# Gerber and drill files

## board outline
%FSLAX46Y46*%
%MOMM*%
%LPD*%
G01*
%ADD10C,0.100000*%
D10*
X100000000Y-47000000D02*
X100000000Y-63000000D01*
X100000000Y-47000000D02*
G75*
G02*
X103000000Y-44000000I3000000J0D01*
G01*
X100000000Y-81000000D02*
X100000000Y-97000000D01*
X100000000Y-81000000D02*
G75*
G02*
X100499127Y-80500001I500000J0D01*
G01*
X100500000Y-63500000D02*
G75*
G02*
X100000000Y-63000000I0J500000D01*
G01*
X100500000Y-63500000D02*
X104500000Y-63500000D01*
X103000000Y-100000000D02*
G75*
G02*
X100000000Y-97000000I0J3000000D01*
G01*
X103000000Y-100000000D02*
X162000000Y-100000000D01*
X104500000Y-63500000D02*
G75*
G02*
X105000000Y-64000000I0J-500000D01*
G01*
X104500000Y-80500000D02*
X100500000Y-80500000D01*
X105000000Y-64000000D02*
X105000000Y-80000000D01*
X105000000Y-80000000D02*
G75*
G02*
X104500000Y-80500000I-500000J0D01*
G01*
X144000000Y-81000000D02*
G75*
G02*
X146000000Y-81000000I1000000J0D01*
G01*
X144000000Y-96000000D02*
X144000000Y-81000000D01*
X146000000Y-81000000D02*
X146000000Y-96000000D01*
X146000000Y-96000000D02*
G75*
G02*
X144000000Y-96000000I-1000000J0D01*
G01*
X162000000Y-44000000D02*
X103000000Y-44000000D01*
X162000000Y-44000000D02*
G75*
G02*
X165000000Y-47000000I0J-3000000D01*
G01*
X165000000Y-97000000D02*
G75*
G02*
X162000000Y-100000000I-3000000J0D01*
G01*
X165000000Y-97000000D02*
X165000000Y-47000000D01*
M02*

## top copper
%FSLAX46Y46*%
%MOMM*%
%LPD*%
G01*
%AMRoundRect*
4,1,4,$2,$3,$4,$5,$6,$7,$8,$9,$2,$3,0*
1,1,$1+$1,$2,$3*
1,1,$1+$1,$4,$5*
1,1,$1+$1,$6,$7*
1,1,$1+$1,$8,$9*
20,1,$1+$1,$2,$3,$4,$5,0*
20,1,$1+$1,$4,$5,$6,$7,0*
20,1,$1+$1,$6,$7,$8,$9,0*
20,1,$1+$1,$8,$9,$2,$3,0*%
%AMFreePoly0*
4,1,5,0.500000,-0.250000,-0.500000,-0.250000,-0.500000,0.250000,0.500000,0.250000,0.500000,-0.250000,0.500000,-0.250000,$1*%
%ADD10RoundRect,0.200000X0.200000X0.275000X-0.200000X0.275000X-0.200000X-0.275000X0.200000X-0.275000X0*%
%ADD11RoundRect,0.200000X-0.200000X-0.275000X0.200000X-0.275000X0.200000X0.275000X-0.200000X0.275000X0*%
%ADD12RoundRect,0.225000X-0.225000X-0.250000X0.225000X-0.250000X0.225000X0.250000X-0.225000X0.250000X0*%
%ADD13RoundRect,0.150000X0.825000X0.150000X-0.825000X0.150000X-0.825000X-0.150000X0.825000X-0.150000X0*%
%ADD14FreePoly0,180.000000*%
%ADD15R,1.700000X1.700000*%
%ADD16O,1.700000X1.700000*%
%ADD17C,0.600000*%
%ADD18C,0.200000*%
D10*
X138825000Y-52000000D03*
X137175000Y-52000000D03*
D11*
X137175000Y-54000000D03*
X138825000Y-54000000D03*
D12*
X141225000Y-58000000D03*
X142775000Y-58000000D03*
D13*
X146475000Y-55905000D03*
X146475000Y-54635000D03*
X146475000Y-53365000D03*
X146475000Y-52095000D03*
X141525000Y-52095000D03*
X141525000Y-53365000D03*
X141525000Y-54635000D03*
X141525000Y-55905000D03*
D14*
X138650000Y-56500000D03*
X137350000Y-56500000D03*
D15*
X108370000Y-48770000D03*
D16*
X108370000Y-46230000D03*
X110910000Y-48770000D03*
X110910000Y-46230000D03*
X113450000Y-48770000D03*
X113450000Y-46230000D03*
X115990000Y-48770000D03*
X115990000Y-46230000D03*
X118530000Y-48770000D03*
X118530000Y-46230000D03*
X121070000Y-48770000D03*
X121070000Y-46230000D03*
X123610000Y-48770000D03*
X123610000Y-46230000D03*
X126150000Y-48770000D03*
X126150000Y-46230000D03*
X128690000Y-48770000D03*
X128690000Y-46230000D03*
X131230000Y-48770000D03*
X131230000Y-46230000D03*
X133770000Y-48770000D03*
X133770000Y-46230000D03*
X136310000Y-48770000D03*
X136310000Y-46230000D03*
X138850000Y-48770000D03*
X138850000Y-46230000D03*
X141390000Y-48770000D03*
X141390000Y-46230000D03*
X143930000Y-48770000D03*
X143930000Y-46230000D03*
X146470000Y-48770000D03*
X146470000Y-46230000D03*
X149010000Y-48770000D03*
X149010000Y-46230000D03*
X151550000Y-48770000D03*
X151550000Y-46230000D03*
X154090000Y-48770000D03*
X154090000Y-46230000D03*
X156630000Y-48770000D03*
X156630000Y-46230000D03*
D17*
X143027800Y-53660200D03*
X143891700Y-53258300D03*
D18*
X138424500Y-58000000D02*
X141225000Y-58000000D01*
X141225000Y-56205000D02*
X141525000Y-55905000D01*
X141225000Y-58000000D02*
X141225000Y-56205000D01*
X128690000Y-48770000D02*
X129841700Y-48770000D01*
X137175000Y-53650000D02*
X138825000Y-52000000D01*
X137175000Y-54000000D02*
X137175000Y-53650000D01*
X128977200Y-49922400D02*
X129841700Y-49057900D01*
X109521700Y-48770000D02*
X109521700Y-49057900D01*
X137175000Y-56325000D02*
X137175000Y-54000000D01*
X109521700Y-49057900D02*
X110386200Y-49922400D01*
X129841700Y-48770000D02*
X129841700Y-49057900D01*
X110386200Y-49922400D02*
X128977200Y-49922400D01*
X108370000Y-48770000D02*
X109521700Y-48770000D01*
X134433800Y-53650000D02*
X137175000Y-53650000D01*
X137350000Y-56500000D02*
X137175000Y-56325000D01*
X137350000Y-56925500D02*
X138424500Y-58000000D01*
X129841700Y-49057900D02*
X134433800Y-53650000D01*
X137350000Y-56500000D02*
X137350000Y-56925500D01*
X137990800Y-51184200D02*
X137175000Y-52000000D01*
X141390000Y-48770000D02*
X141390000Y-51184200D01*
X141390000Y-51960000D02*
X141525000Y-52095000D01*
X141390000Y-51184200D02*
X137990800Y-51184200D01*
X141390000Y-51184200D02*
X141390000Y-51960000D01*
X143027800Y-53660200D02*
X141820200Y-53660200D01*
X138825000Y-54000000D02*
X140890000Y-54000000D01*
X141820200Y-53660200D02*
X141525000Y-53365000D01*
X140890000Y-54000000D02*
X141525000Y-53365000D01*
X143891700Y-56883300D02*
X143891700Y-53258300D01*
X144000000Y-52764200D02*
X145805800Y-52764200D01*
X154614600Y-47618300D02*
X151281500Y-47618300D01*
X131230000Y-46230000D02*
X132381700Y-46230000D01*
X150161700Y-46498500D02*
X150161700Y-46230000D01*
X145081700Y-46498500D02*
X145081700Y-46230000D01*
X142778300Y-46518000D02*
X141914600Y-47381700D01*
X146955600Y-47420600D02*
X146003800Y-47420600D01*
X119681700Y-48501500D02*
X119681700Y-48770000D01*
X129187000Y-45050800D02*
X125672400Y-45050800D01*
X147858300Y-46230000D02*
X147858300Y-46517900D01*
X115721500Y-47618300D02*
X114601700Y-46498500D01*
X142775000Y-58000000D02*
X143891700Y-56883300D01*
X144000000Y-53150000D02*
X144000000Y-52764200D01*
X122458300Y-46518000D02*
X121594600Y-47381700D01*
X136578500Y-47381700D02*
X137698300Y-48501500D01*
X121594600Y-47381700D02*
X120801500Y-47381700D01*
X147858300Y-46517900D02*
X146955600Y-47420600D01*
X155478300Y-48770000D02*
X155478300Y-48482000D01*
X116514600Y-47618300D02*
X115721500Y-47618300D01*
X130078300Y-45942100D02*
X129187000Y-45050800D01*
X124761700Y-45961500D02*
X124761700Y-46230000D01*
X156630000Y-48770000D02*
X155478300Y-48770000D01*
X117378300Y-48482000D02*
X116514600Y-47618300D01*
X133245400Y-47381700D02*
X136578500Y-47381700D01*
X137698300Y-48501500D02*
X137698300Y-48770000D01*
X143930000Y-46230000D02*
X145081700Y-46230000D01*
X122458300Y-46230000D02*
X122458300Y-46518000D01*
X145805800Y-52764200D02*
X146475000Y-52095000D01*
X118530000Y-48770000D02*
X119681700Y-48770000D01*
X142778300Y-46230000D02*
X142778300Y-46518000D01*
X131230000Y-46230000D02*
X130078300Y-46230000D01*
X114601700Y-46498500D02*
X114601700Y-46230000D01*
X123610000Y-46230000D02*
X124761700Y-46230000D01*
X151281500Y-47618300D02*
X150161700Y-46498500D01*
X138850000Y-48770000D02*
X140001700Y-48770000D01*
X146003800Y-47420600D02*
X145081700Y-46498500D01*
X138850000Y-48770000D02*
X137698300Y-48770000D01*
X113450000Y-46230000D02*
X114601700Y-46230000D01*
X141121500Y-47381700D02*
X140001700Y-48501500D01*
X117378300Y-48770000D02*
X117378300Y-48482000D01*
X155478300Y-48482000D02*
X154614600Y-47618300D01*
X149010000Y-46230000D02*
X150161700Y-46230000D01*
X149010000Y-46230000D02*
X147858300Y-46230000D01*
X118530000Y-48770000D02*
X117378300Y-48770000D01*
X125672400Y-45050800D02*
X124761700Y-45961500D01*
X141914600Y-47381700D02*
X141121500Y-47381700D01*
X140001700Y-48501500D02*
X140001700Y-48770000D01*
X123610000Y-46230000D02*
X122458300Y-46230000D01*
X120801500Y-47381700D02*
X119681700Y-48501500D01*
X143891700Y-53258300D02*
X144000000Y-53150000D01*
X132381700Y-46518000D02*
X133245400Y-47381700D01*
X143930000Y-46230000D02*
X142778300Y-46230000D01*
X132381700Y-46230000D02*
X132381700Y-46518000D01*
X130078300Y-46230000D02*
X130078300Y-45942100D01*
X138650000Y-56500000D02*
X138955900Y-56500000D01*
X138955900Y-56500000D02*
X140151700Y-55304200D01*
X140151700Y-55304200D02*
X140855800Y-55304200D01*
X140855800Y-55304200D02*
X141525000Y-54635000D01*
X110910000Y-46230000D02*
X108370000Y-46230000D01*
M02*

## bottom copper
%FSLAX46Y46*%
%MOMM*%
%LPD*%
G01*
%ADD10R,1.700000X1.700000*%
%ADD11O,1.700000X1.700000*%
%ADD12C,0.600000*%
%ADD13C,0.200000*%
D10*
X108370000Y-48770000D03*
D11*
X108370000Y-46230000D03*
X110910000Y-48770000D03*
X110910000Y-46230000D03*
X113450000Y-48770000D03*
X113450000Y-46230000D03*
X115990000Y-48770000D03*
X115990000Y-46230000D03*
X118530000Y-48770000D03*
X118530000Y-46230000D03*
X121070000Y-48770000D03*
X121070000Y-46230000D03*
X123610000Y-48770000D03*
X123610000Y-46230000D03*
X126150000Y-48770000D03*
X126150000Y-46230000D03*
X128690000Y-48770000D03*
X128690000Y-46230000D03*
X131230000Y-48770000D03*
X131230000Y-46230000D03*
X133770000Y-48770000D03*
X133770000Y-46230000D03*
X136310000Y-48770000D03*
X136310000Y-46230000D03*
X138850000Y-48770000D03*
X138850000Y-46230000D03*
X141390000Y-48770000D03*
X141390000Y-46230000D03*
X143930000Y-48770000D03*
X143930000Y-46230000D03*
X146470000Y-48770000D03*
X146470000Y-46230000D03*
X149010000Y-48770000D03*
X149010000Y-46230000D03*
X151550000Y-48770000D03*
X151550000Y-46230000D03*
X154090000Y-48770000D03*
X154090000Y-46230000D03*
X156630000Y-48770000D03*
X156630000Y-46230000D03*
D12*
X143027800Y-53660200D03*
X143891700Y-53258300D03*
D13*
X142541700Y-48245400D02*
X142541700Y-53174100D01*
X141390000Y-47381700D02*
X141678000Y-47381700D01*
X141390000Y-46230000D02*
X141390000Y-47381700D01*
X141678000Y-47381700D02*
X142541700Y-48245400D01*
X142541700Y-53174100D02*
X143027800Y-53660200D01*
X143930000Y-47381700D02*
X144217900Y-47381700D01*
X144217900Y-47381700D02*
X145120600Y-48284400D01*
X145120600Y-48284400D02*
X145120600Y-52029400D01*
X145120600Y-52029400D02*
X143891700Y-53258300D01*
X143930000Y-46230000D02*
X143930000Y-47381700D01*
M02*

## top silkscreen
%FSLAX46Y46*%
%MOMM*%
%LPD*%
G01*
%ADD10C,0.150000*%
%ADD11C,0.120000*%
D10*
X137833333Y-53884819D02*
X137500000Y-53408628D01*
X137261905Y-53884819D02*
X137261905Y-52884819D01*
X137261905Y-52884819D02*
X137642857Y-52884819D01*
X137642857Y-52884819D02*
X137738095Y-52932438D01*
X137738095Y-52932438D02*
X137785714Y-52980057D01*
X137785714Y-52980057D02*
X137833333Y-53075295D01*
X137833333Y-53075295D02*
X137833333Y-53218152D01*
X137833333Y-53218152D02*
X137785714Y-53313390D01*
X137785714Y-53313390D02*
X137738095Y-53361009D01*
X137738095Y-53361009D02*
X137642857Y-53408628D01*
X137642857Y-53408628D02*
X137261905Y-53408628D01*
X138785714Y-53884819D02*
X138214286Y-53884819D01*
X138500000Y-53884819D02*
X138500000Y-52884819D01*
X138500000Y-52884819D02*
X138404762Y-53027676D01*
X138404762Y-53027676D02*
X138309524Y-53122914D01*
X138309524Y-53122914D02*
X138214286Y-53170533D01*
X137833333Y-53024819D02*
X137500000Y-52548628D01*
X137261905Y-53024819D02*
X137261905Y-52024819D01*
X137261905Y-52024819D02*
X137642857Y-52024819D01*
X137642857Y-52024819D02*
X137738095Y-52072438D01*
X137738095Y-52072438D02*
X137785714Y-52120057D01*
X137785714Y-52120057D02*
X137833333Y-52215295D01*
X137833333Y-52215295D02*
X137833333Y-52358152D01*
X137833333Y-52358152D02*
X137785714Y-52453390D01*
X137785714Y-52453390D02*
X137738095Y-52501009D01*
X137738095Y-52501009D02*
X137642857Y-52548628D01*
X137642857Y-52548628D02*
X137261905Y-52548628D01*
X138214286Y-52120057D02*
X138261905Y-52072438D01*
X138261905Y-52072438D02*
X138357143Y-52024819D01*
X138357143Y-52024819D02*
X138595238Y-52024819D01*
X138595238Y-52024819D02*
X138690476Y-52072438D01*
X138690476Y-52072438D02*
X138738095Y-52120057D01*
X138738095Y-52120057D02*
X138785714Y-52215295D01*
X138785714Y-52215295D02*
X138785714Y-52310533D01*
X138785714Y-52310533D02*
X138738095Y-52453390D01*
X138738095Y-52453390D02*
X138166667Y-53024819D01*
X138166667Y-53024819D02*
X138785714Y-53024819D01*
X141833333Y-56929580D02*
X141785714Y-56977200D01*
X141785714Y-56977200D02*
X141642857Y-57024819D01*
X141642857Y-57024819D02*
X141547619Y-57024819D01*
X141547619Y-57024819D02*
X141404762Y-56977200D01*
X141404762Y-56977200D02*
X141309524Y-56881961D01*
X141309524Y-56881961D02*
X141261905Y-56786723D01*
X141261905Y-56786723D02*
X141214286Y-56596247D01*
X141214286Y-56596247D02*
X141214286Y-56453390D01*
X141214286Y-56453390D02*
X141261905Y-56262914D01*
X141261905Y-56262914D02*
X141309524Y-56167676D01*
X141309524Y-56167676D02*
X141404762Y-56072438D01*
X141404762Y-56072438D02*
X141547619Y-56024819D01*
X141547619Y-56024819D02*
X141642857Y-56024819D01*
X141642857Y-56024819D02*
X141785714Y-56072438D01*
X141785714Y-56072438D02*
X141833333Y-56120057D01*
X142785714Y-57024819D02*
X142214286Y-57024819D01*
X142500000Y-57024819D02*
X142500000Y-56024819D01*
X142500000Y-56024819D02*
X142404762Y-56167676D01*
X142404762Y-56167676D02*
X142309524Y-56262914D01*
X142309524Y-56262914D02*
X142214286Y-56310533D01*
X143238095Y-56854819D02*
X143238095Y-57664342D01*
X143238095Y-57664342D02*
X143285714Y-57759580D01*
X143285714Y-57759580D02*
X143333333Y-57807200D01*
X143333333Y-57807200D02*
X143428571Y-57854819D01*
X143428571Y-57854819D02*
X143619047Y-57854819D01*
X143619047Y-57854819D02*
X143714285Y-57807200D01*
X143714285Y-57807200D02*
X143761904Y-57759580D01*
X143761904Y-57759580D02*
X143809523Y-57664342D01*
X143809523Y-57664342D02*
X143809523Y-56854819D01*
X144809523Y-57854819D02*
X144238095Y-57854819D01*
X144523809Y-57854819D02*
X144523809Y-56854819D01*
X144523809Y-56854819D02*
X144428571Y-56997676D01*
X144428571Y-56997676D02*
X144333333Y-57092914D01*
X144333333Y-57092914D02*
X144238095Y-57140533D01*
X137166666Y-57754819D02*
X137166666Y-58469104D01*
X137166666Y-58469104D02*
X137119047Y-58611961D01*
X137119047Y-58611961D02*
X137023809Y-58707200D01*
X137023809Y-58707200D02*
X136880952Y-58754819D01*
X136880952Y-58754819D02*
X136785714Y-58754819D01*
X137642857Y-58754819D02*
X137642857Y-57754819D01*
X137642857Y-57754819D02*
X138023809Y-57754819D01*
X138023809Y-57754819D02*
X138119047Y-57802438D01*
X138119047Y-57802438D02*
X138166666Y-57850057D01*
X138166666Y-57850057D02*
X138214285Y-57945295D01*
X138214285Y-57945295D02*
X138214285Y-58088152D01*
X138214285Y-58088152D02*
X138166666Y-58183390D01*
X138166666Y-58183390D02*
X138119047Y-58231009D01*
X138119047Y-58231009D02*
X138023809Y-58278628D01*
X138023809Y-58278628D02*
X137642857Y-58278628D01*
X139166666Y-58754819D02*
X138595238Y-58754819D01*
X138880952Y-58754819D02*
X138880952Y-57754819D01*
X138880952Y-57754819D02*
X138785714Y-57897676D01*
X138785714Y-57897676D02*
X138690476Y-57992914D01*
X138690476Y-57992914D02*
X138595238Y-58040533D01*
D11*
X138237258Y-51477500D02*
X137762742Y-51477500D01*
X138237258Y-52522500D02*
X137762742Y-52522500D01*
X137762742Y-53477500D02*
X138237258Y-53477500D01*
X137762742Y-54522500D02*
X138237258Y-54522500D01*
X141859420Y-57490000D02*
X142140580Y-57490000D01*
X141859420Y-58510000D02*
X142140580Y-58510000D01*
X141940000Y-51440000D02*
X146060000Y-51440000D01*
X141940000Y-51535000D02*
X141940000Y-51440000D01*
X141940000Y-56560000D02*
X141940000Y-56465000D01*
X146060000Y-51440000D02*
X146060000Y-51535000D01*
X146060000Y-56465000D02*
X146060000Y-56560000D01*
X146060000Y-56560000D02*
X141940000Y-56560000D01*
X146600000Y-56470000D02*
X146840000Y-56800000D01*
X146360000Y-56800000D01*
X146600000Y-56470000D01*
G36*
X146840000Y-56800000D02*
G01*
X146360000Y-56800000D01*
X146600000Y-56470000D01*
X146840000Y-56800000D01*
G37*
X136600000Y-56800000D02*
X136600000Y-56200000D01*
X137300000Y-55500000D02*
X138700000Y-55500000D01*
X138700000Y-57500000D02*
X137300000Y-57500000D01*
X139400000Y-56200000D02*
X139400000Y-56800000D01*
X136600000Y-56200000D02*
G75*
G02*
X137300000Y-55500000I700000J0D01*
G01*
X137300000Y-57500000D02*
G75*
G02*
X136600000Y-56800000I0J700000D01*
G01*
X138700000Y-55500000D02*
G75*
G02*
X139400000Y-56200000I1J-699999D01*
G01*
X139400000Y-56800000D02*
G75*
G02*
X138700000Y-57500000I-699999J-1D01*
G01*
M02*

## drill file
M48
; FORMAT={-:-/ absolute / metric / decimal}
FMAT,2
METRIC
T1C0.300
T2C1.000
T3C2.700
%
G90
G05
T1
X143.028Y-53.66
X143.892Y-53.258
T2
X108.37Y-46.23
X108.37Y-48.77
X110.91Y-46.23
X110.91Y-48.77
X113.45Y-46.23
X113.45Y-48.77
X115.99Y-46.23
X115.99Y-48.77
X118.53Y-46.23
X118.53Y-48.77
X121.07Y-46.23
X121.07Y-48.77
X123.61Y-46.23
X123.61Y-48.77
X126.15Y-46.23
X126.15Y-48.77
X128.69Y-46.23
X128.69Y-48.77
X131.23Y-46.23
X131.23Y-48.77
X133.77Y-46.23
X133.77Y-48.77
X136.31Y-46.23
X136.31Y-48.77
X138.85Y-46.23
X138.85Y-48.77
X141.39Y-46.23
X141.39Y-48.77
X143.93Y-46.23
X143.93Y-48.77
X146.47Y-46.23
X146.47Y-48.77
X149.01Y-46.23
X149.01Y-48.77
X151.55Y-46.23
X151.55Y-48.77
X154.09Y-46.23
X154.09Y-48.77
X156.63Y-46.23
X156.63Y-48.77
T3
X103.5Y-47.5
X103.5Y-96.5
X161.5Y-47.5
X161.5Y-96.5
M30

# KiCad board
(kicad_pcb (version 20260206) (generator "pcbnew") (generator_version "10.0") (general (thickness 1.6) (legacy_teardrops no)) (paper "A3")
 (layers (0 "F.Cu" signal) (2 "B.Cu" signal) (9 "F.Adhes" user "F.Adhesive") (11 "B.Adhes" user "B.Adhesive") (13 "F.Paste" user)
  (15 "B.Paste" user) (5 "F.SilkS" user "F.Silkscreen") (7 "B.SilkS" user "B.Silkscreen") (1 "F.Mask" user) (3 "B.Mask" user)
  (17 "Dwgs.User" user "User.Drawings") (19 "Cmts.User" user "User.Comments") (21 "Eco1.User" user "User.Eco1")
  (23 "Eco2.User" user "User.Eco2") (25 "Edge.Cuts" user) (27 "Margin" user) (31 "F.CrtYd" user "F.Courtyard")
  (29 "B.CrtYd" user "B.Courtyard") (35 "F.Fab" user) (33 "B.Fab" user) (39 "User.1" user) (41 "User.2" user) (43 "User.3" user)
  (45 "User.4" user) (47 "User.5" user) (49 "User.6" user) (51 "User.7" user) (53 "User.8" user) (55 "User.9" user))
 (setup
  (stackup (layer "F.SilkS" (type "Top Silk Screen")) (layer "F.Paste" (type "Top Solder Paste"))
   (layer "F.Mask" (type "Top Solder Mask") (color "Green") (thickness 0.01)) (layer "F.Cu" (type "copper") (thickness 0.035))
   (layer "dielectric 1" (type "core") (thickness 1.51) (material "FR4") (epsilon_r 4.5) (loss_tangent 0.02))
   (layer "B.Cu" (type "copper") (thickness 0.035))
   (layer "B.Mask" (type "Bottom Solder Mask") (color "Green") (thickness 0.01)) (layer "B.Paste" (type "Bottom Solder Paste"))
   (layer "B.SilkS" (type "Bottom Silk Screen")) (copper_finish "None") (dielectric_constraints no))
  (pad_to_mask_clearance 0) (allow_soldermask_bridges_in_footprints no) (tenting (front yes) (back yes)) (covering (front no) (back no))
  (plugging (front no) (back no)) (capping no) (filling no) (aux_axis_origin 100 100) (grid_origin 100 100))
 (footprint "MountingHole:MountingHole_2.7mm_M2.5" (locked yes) (layer "F.Cu") (at 161.5 47.5)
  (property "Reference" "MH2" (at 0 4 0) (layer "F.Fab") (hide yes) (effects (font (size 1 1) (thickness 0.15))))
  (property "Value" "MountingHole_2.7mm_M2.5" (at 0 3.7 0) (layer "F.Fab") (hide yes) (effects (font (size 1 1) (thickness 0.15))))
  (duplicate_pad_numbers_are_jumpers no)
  (pad "" np_thru_hole circle (at 0 0) (size 2.7 2.7) (drill 2.7) (layers "*.Cu" "*.Mask")))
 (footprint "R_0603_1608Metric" (layer "F.Cu") (at 138 52 180)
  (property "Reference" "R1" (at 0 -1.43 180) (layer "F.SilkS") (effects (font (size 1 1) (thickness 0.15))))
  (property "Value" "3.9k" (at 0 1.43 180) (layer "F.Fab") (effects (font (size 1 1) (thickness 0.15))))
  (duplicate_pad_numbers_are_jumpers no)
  (fp_line (start -0.237258 0.5225) (end 0.237258 0.5225) (stroke (width 0.12) (type solid)) (layer "F.SilkS"))
  (fp_line (start -0.237258 -0.5225) (end 0.237258 -0.5225) (stroke (width 0.12) (type solid)) (layer "F.SilkS"))
  (pad "1" smd roundrect (at -0.825 0 180) (size 0.8 0.95) (layers "F.Cu" "F.Mask" "F.Paste") (roundrect_rratio 0.25) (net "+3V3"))
  (pad "2" smd roundrect (at 0.825 0 180) (size 0.8 0.95) (layers "F.Cu" "F.Mask" "F.Paste") (roundrect_rratio 0.25) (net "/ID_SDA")))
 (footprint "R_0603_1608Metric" (layer "F.Cu") (at 138 54)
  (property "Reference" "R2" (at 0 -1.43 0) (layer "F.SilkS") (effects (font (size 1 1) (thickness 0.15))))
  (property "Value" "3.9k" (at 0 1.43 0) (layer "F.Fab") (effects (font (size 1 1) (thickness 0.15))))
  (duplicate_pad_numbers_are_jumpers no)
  (fp_line (start -0.237258 -0.5225) (end 0.237258 -0.5225) (stroke (width 0.12) (type solid)) (layer "F.SilkS"))
  (fp_line (start -0.237258 0.5225) (end 0.237258 0.5225) (stroke (width 0.12) (type solid)) (layer "F.SilkS"))
  (pad "1" smd roundrect (at -0.825 0) (size 0.8 0.95) (layers "F.Cu" "F.Mask" "F.Paste") (roundrect_rratio 0.25) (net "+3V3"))
  (pad "2" smd roundrect (at 0.825 0) (size 0.8 0.95) (layers "F.Cu" "F.Mask" "F.Paste") (roundrect_rratio 0.25) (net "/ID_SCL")))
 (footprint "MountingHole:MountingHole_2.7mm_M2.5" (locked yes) (layer "F.Cu") (at 103.5 96.5)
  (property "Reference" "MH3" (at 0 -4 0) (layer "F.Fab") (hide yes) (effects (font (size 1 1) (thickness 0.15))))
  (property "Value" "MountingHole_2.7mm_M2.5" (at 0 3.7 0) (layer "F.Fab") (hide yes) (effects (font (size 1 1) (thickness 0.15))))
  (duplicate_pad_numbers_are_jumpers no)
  (pad "" np_thru_hole circle (at 0 0) (size 2.7 2.7) (drill 2.7) (layers "*.Cu" "*.Mask")))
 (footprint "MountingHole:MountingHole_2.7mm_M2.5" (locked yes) (layer "F.Cu") (at 103.5 47.5)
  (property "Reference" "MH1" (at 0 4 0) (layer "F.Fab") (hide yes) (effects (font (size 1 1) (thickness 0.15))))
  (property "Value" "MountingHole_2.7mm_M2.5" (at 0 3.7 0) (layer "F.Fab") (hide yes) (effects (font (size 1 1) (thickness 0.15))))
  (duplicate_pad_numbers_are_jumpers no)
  (pad "" np_thru_hole circle (at 0 0) (size 2.7 2.7) (drill 2.7) (layers "*.Cu" "*.Mask")))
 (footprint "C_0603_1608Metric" (layer "F.Cu") (at 142 58)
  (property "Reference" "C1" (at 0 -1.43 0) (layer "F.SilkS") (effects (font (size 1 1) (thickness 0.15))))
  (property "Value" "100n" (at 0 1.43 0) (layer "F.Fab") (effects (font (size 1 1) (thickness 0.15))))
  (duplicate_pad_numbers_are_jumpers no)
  (fp_line (start -0.14058 -0.51) (end 0.14058 -0.51) (stroke (width 0.12) (type solid)) (layer "F.SilkS"))
  (fp_line (start -0.14058 0.51) (end 0.14058 0.51) (stroke (width 0.12) (type solid)) (layer "F.SilkS"))
  (pad "1" smd roundrect (at -0.775 0) (size 0.9 0.95) (layers "F.Cu" "F.Mask" "F.Paste") (roundrect_rratio 0.25) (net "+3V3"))
  (pad "2" smd roundrect (at 0.775 0) (size 0.9 0.95) (layers "F.Cu" "F.Mask" "F.Paste") (roundrect_rratio 0.25) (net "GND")))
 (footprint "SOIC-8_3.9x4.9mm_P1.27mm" (layer "F.Cu") (at 144 54 180)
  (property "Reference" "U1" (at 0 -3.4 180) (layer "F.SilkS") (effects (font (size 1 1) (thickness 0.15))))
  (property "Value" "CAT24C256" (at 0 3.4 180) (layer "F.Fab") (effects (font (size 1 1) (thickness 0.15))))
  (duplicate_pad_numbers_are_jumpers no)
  (fp_line (start 2.06 2.56) (end -2.06 2.56) (stroke (width 0.12) (type solid)) (layer "F.SilkS"))
  (fp_line (start 2.06 2.465) (end 2.06 2.56) (stroke (width 0.12) (type solid)) (layer "F.SilkS"))
  (fp_line (start 2.06 -2.56) (end 2.06 -2.465) (stroke (width 0.12) (type solid)) (layer "F.SilkS"))
  (fp_line (start -2.06 2.56) (end -2.06 2.465) (stroke (width 0.12) (type solid)) (layer "F.SilkS"))
  (fp_line (start -2.06 -2.465) (end -2.06 -2.56) (stroke (width 0.12) (type solid)) (layer "F.SilkS"))
  (fp_line (start -2.06 -2.56) (end 2.06 -2.56) (stroke (width 0.12) (type solid)) (layer "F.SilkS"))
  (fp_poly (pts (xy -2.6 -2.47) (xy -2.84 -2.8) (xy -2.36 -2.8)) (stroke (width 0.12) (type solid)) (fill yes) (layer "F.SilkS"))
  (pad "1" smd roundrect (at -2.475 -1.905 180) (size 1.95 0.6) (layers "F.Cu" "F.Mask" "F.Paste") (roundrect_rratio 0.25)
   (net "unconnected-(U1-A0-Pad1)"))
  (pad "2" smd roundrect (at -2.475 -0.635 180) (size 1.95 0.6) (layers "F.Cu" "F.Mask" "F.Paste") (roundrect_rratio 0.25)
   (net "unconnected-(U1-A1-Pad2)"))
  (pad "3" smd roundrect (at -2.475 0.635 180) (size 1.95 0.6) (layers "F.Cu" "F.Mask" "F.Paste") (roundrect_rratio 0.25)
   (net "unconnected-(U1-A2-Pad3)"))
  (pad "4" smd roundrect (at -2.475 1.905 180) (size 1.95 0.6) (layers "F.Cu" "F.Mask" "F.Paste") (roundrect_rratio 0.25) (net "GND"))
  (pad "5" smd roundrect (at 2.475 1.905 180) (size 1.95 0.6) (layers "F.Cu" "F.Mask" "F.Paste") (roundrect_rratio 0.25) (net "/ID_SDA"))
  (pad "6" smd roundrect (at 2.475 0.635 180) (size 1.95 0.6) (layers "F.Cu" "F.Mask" "F.Paste") (roundrect_rratio 0.25) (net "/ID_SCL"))
  (pad "7" smd roundrect (at 2.475 -0.635 180) (size 1.95 0.6) (layers "F.Cu" "F.Mask" "F.Paste") (roundrect_rratio 0.25)
   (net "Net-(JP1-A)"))
  (pad "8" smd roundrect (at 2.475 -1.905 180) (size 1.95 0.6) (layers "F.Cu" "F.Mask" "F.Paste") (roundrect_rratio 0.25) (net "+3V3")))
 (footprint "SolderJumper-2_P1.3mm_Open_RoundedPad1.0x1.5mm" (layer "F.Cu") (at 138 56.5 180)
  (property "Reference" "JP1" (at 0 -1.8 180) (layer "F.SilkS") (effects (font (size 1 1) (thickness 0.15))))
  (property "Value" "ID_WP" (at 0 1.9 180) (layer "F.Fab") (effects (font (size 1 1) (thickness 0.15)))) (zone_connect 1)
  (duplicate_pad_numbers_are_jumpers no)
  (fp_line (start 1.4 -0.3) (end 1.4 0.3) (stroke (width 0.12) (type solid)) (layer "F.SilkS"))
  (fp_line (start 0.7 1) (end -0.7 1) (stroke (width 0.12) (type solid)) (layer "F.SilkS"))
  (fp_line (start -0.7 -1) (end 0.7 -1) (stroke (width 0.12) (type solid)) (layer "F.SilkS"))
  (fp_line (start -1.4 0.3) (end -1.4 -0.3) (stroke (width 0.12) (type solid)) (layer "F.SilkS"))
  (fp_arc (start 1.4 0.3) (mid 1.194975 0.794975) (end 0.7 1) (stroke (width 0.12) (type solid)) (layer "F.SilkS"))
  (fp_arc (start 0.7 -1) (mid 1.194975 -0.794975) (end 1.4 -0.3) (stroke (width 0.12) (type solid)) (layer "F.SilkS"))
  (fp_arc (start -0.7 1) (mid -1.194975 0.794975) (end -1.4 0.3) (stroke (width 0.12) (type solid)) (layer "F.SilkS"))
  (fp_arc (start -1.4 -0.3) (mid -1.194975 -0.794975) (end -0.7 -1) (stroke (width 0.12) (type solid)) (layer "F.SilkS"))
  (pad "1" smd custom (at -0.65 0 180) (size 1 0.5) (layers "F.Cu" "F.Mask") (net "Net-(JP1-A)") (zone_connect 2) (thermal_bridge_angle 45)
   (options (clearance outline) (anchor rect)) (primitives))
  (pad "2" smd custom (at 0.65 0 180) (size 1 0.5) (layers "F.Cu" "F.Mask") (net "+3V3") (zone_connect 2) (thermal_bridge_angle 45)
   (options (clearance outline) (anchor rect)) (primitives)))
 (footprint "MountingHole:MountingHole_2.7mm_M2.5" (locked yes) (layer "F.Cu") (at 161.5 96.5)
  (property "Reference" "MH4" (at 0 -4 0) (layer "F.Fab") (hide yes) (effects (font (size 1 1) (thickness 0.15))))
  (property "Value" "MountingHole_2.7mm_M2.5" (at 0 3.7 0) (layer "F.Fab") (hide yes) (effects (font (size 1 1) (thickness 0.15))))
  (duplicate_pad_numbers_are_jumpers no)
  (pad "" np_thru_hole circle (at 0 0) (size 2.7 2.7) (drill 2.7) (layers "*.Cu" "*.Mask")))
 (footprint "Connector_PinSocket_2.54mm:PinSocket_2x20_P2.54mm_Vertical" (layer "B.Cu") (at 108.37 48.77 -90)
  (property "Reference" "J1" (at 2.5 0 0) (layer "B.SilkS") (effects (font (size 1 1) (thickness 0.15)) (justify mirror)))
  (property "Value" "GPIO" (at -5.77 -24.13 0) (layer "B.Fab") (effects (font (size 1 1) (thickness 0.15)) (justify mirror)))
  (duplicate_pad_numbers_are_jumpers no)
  (pad "1" thru_hole rect (at 0 0 270) (size 1.7 1.7) (drill 1) (layers "*.Cu" "*.Mask") (remove_unused_layers no) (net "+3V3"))
  (pad "2" thru_hole oval (at -2.54 0 270) (size 1.7 1.7) (drill 1) (layers "*.Cu" "*.Mask") (remove_unused_layers no) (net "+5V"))
  (pad "3" thru_hole oval (at 0 -2.54 270) (size 1.7 1.7) (drill 1) (layers "*.Cu" "*.Mask") (remove_unused_layers no)
   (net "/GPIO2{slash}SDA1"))
  (pad "4" thru_hole oval (at -2.54 -2.54 270) (size 1.7 1.7) (drill 1) (layers "*.Cu" "*.Mask") (remove_unused_layers no) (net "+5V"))
  (pad "5" thru_hole oval (at 0 -5.08 270) (size 1.7 1.7) (drill 1) (layers "*.Cu" "*.Mask") (remove_unused_layers no)
   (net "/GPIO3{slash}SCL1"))
  (pad "6" thru_hole oval (at -2.54 -5.08 270) (size 1.7 1.7) (drill 1) (layers "*.Cu" "*.Mask") (remove_unused_layers no) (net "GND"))
  (pad "7" thru_hole oval (at 0 -7.62 270) (size 1.7 1.7) (drill 1) (layers "*.Cu" "*.Mask") (remove_unused_layers no)
   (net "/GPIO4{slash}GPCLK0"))
  (pad "8" thru_hole oval (at -2.54 -7.62 270) (size 1.7 1.7) (drill 1) (layers "*.Cu" "*.Mask") (remove_unused_layers no)
   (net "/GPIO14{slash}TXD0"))
  (pad "9" thru_hole oval (at 0 -10.16 270) (size 1.7 1.7) (drill 1) (layers "*.Cu" "*.Mask") (remove_unused_layers no) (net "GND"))
  (pad "10" thru_hole oval (at -2.54 -10.16 270) (size 1.7 1.7) (drill 1) (layers "*.Cu" "*.Mask") (remove_unused_layers no)
   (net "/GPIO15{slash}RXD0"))
  (pad "11" thru_hole oval (at 0 -12.7 270) (size 1.7 1.7) (drill 1) (layers "*.Cu" "*.Mask") (remove_unused_layers no) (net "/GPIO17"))
  (pad "12" thru_hole oval (at -2.54 -12.7 270) (size 1.7 1.7) (drill 1) (layers "*.Cu" "*.Mask") (remove_unused_layers no)
   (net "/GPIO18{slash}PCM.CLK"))
  (pad "13" thru_hole oval (at 0 -15.24 270) (size 1.7 1.7) (drill 1) (layers "*.Cu" "*.Mask") (remove_unused_layers no) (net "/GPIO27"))
  (pad "14" thru_hole oval (at -2.54 -15.24 270) (size 1.7 1.7) (drill 1) (layers "*.Cu" "*.Mask") (remove_unused_layers no) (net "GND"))
  (pad "15" thru_hole oval (at 0 -17.78 270) (size 1.7 1.7) (drill 1) (layers "*.Cu" "*.Mask") (remove_unused_layers no) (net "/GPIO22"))
  (pad "16" thru_hole oval (at -2.54 -17.78 270) (size 1.7 1.7) (drill 1) (layers "*.Cu" "*.Mask") (remove_unused_layers no) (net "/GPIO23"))
  (pad "17" thru_hole oval (at 0 -20.32 270) (size 1.7 1.7) (drill 1) (layers "*.Cu" "*.Mask") (remove_unused_layers no) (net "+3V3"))
  (pad "18" thru_hole oval (at -2.54 -20.32 270) (size 1.7 1.7) (drill 1) (layers "*.Cu" "*.Mask") (remove_unused_layers no) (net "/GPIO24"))
  (pad "19" thru_hole oval (at 0 -22.86 270) (size 1.7 1.7) (drill 1) (layers "*.Cu" "*.Mask") (remove_unused_layers no)
   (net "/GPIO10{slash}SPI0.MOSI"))
  (pad "20" thru_hole oval (at -2.54 -22.86 270) (size 1.7 1.7) (drill 1) (layers "*.Cu" "*.Mask") (remove_unused_layers no) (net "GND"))
  (pad "21" thru_hole oval (at 0 -25.4 270) (size 1.7 1.7) (drill 1) (layers "*.Cu" "*.Mask") (remove_unused_layers no)
   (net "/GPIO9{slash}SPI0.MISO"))
  (pad "22" thru_hole oval (at -2.54 -25.4 270) (size 1.7 1.7) (drill 1) (layers "*.Cu" "*.Mask") (remove_unused_layers no) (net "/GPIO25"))
  (pad "23" thru_hole oval (at 0 -27.94 270) (size 1.7 1.7) (drill 1) (layers "*.Cu" "*.Mask") (remove_unused_layers no)
   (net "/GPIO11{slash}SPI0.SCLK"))
  (pad "24" thru_hole oval (at -2.54 -27.94 270) (size 1.7 1.7) (drill 1) (layers "*.Cu" "*.Mask") (remove_unused_layers no)
   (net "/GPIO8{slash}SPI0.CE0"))
  (pad "25" thru_hole oval (at 0 -30.48 270) (size 1.7 1.7) (drill 1) (layers "*.Cu" "*.Mask") (remove_unused_layers no) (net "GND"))
  (pad "26" thru_hole oval (at -2.54 -30.48 270) (size 1.7 1.7) (drill 1) (layers "*.Cu" "*.Mask") (remove_unused_layers no)
   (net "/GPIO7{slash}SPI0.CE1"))
  (pad "27" thru_hole oval (at 0 -33.02 270) (size 1.7 1.7) (drill 1) (layers "*.Cu" "*.Mask") (remove_unused_layers no) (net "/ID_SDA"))
  (pad "28" thru_hole oval (at -2.54 -33.02 270) (size 1.7 1.7) (drill 1) (layers "*.Cu" "*.Mask") (remove_unused_layers no) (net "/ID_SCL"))
  (pad "29" thru_hole oval (at 0 -35.56 270) (size 1.7 1.7) (drill 1) (layers "*.Cu" "*.Mask") (remove_unused_layers no) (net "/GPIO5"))
  (pad "30" thru_hole oval (at -2.54 -35.56 270) (size 1.7 1.7) (drill 1) (layers "*.Cu" "*.Mask") (remove_unused_layers no) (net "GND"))
  (pad "31" thru_hole oval (at 0 -38.1 270) (size 1.7 1.7) (drill 1) (layers "*.Cu" "*.Mask") (remove_unused_layers no) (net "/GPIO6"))
  (pad "32" thru_hole oval (at -2.54 -38.1 270) (size 1.7 1.7) (drill 1) (layers "*.Cu" "*.Mask") (remove_unused_layers no)
   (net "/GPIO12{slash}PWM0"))
  (pad "33" thru_hole oval (at 0 -40.64 270) (size 1.7 1.7) (drill 1) (layers "*.Cu" "*.Mask") (remove_unused_layers no)
   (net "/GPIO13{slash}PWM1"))
  (pad "34" thru_hole oval (at -2.54 -40.64 270) (size 1.7 1.7) (drill 1) (layers "*.Cu" "*.Mask") (remove_unused_layers no) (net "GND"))
  (pad "35" thru_hole oval (at 0 -43.18 270) (size 1.7 1.7) (drill 1) (layers "*.Cu" "*.Mask") (remove_unused_layers no)
   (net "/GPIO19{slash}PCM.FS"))
  (pad "36" thru_hole oval (at -2.54 -43.18 270) (size 1.7 1.7) (drill 1) (layers "*.Cu" "*.Mask") (remove_unused_layers no) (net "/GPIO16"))
  (pad "37" thru_hole oval (at 0 -45.72 270) (size 1.7 1.7) (drill 1) (layers "*.Cu" "*.Mask") (remove_unused_layers no) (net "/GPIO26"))
  (pad "38" thru_hole oval (at -2.54 -45.72 270) (size 1.7 1.7) (drill 1) (layers "*.Cu" "*.Mask") (remove_unused_layers no)
   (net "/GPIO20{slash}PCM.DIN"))
  (pad "39" thru_hole oval (at 0 -48.26 270) (size 1.7 1.7) (drill 1) (layers "*.Cu" "*.Mask") (remove_unused_layers no) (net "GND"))
  (pad "40" thru_hole oval (at -2.54 -48.26 270) (size 1.7 1.7) (drill 1) (layers "*.Cu" "*.Mask") (remove_unused_layers no)
   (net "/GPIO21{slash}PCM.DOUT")))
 (gr_line (start 100 47) (end 100 63) (stroke (width 0.1) (type solid)) (layer "Edge.Cuts"))
 (gr_arc (start 100 47) (mid 100.87868 44.87868) (end 103 44) (stroke (width 0.1) (type solid)) (layer "Edge.Cuts"))
 (gr_line (start 100 81) (end 100 97) (stroke (width 0.1) (type solid)) (layer "Edge.Cuts"))
 (gr_arc (start 100 81) (mid 100.146138 80.646755) (end 100.499127 80.500001) (stroke (width 0.1) (type solid)) (layer "Edge.Cuts"))
 (gr_arc (start 100.5 63.5) (mid 100.146447 63.353553) (end 100 63) (stroke (width 0.1) (type solid)) (layer "Edge.Cuts"))
 (gr_line (start 100.5 63.5) (end 104.5 63.5) (stroke (width 0.1) (type solid)) (layer "Edge.Cuts"))
 (gr_arc (start 103 100) (mid 100.87868 99.12132) (end 100 97) (stroke (width 0.1) (type solid)) (layer "Edge.Cuts"))
 (gr_line (start 103 100) (end 162 100) (stroke (width 0.1) (type solid)) (layer "Edge.Cuts"))
 (gr_arc (start 104.5 63.5) (mid 104.853553 63.646447) (end 105 64) (stroke (width 0.1) (type solid)) (layer "Edge.Cuts"))
 (gr_line (start 104.5 80.5) (end 100.5 80.5) (stroke (width 0.1) (type solid)) (layer "Edge.Cuts"))
 (gr_line (start 105 64) (end 105 80) (stroke (width 0.1) (type solid)) (layer "Edge.Cuts"))
 (gr_arc (start 105 80) (mid 104.853553 80.353553) (end 104.5 80.5) (stroke (width 0.1) (type solid)) (layer "Edge.Cuts"))
 (gr_arc (start 144 81) (mid 145 80) (end 146 81) (stroke (width 0.1) (type solid)) (layer "Edge.Cuts"))
 (gr_line (start 144 96) (end 144 81) (stroke (width 0.1) (type solid)) (layer "Edge.Cuts"))
 (gr_line (start 146 81) (end 146 96) (stroke (width 0.1) (type solid)) (layer "Edge.Cuts"))
 (gr_arc (start 146 96) (mid 145 97) (end 144 96) (stroke (width 0.1) (type solid)) (layer "Edge.Cuts"))
 (gr_line (start 162 44) (end 103 44) (stroke (width 0.1) (type solid)) (layer "Edge.Cuts"))
 (gr_arc (start 162 44) (mid 164.12132 44.87868) (end 165 47) (stroke (width 0.1) (type solid)) (layer "Edge.Cuts"))
 (gr_arc (start 165 97) (mid 164.12132 99.12132) (end 162 100) (stroke (width 0.1) (type solid)) (layer "Edge.Cuts"))
 (gr_line (start 165 97) (end 165 47) (stroke (width 0.1) (type solid)) (layer "Edge.Cuts"))
 (segment (start 138.4245 58) (end 141.225 58) (width 0.2) (layer "F.Cu") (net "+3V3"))
 (segment (start 141.225 56.205) (end 141.525 55.905) (width 0.2) (layer "F.Cu") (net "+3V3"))
 (segment (start 141.225 58) (end 141.225 56.205) (width 0.2) (layer "F.Cu") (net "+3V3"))
 (segment (start 128.69 48.77) (end 129.8417 48.77) (width 0.2) (layer "F.Cu") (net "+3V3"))
 (segment (start 137.175 53.65) (end 138.825 52) (width 0.2) (layer "F.Cu") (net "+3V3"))
 (segment (start 137.175 54) (end 137.175 53.65) (width 0.2) (layer "F.Cu") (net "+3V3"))
 (segment (start 128.9772 49.9224) (end 129.8417 49.0579) (width 0.2) (layer "F.Cu") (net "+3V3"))
 (segment (start 109.5217 48.77) (end 109.5217 49.0579) (width 0.2) (layer "F.Cu") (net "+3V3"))
 (segment (start 137.175 56.325) (end 137.175 54) (width 0.2) (layer "F.Cu") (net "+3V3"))
 (segment (start 109.5217 49.0579) (end 110.3862 49.9224) (width 0.2) (layer "F.Cu") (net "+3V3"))
 (segment (start 129.8417 48.77) (end 129.8417 49.0579) (width 0.2) (layer "F.Cu") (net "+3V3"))
 (segment (start 110.3862 49.9224) (end 128.9772 49.9224) (width 0.2) (layer "F.Cu") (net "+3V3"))
 (segment (start 108.37 48.77) (end 109.5217 48.77) (width 0.2) (layer "F.Cu") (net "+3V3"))
 (segment (start 134.4338 53.65) (end 137.175 53.65) (width 0.2) (layer "F.Cu") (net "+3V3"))
 (segment (start 137.35 56.5) (end 137.175 56.325) (width 0.2) (layer "F.Cu") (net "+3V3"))
 (segment (start 137.35 56.9255) (end 138.4245 58) (width 0.2) (layer "F.Cu") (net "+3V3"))
 (segment (start 129.8417 49.0579) (end 134.4338 53.65) (width 0.2) (layer "F.Cu") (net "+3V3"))
 (segment (start 137.35 56.5) (end 137.35 56.9255) (width 0.2) (layer "F.Cu") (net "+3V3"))
 (segment (start 137.9908 51.1842) (end 137.175 52) (width 0.2) (layer "F.Cu") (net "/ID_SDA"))
 (segment (start 141.39 48.77) (end 141.39 51.1842) (width 0.2) (layer "F.Cu") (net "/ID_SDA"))
 (segment (start 141.39 51.96) (end 141.525 52.095) (width 0.2) (layer "F.Cu") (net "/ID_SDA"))
 (segment (start 141.39 51.1842) (end 137.9908 51.1842) (width 0.2) (layer "F.Cu") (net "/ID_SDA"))
 (segment (start 141.39 51.1842) (end 141.39 51.96) (width 0.2) (layer "F.Cu") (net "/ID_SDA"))
 (segment (start 143.0278 53.6602) (end 141.8202 53.6602) (width 0.2) (layer "F.Cu") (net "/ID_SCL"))
 (segment (start 138.825 54) (end 140.89 54) (width 0.2) (layer "F.Cu") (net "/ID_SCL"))
 (segment (start 141.8202 53.6602) (end 141.525 53.365) (width 0.2) (layer "F.Cu") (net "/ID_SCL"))
 (segment (start 140.89 54) (end 141.525 53.365) (width 0.2) (layer "F.Cu") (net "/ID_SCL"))
 (via (at 143.0278 53.6602) (size 0.6) (drill 0.3) (layers "F.Cu" "B.Cu") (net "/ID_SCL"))
 (segment (start 142.5417 48.2454) (end 142.5417 53.1741) (width 0.2) (layer "B.Cu") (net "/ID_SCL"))
 (segment (start 141.39 47.3817) (end 141.678 47.3817) (width 0.2) (layer "B.Cu") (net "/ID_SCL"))
 (segment (start 141.39 46.23) (end 141.39 47.3817) (width 0.2) (layer "B.Cu") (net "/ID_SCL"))
 (segment (start 141.678 47.3817) (end 142.5417 48.2454) (width 0.2) (layer "B.Cu") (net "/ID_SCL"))
 (segment (start 142.5417 53.1741) (end 143.0278 53.6602) (width 0.2) (layer "B.Cu") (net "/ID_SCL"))
 (segment (start 143.8917 56.8833) (end 143.8917 53.2583) (width 0.2) (layer "F.Cu") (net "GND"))
 (segment (start 144 52.7642) (end 145.8058 52.7642) (width 0.2) (layer "F.Cu") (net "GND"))
 (segment (start 154.6146 47.6183) (end 151.2815 47.6183) (width 0.2) (layer "F.Cu") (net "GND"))
 (segment (start 131.23 46.23) (end 132.3817 46.23) (width 0.2) (layer "F.Cu") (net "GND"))
 (segment (start 150.1617 46.4985) (end 150.1617 46.23) (width 0.2) (layer "F.Cu") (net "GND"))
 (segment (start 145.0817 46.4985) (end 145.0817 46.23) (width 0.2) (layer "F.Cu") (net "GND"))
 (segment (start 142.7783 46.518) (end 141.9146 47.3817) (width 0.2) (layer "F.Cu") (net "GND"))
 (segment (start 146.9556 47.4206) (end 146.0038 47.4206) (width 0.2) (layer "F.Cu") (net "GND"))
 (segment (start 119.6817 48.5015) (end 119.6817 48.77) (width 0.2) (layer "F.Cu") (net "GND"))
 (segment (start 129.187 45.0508) (end 125.6724 45.0508) (width 0.2) (layer "F.Cu") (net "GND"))
 (segment (start 147.8583 46.23) (end 147.8583 46.5179) (width 0.2) (layer "F.Cu") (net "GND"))
 (segment (start 115.7215 47.6183) (end 114.6017 46.4985) (width 0.2) (layer "F.Cu") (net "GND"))
 (segment (start 142.775 58) (end 143.8917 56.8833) (width 0.2) (layer "F.Cu") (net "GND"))
 (segment (start 144 53.15) (end 144 52.7642) (width 0.2) (layer "F.Cu") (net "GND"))
 (segment (start 122.4583 46.518) (end 121.5946 47.3817) (width 0.2) (layer "F.Cu") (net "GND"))
 (segment (start 136.5785 47.3817) (end 137.6983 48.5015) (width 0.2) (layer "F.Cu") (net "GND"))
 (segment (start 121.5946 47.3817) (end 120.8015 47.3817) (width 0.2) (layer "F.Cu") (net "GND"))
 (segment (start 147.8583 46.5179) (end 146.9556 47.4206) (width 0.2) (layer "F.Cu") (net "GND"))
 (segment (start 155.4783 48.77) (end 155.4783 48.482) (width 0.2) (layer "F.Cu") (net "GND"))
 (segment (start 116.5146 47.6183) (end 115.7215 47.6183) (width 0.2) (layer "F.Cu") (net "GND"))
 (segment (start 130.0783 45.9421) (end 129.187 45.0508) (width 0.2) (layer "F.Cu") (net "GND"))
 (segment (start 124.7617 45.9615) (end 124.7617 46.23) (width 0.2) (layer "F.Cu") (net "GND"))
 (segment (start 156.63 48.77) (end 155.4783 48.77) (width 0.2) (layer "F.Cu") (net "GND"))
 (segment (start 117.3783 48.482) (end 116.5146 47.6183) (width 0.2) (layer "F.Cu") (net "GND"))
 (segment (start 133.2454 47.3817) (end 136.5785 47.3817) (width 0.2) (layer "F.Cu") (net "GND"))
 (segment (start 137.6983 48.5015) (end 137.6983 48.77) (width 0.2) (layer "F.Cu") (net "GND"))
 (segment (start 143.93 46.23) (end 145.0817 46.23) (width 0.2) (layer "F.Cu") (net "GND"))
 (segment (start 122.4583 46.23) (end 122.4583 46.518) (width 0.2) (layer "F.Cu") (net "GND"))
 (segment (start 145.8058 52.7642) (end 146.475 52.095) (width 0.2) (layer "F.Cu") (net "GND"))
 (segment (start 118.53 48.77) (end 119.6817 48.77) (width 0.2) (layer "F.Cu") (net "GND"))
 (segment (start 142.7783 46.23) (end 142.7783 46.518) (width 0.2) (layer "F.Cu") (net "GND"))
 (segment (start 131.23 46.23) (end 130.0783 46.23) (width 0.2) (layer "F.Cu") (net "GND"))
 (segment (start 114.6017 46.4985) (end 114.6017 46.23) (width 0.2) (layer "F.Cu") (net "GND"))
 (segment (start 123.61 46.23) (end 124.7617 46.23) (width 0.2) (layer "F.Cu") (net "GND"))
 (segment (start 151.2815 47.6183) (end 150.1617 46.4985) (width 0.2) (layer "F.Cu") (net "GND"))
 (segment (start 138.85 48.77) (end 140.0017 48.77) (width 0.2) (layer "F.Cu") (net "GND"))
 (segment (start 146.0038 47.4206) (end 145.0817 46.4985) (width 0.2) (layer "F.Cu") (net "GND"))
 (segment (start 138.85 48.77) (end 137.6983 48.77) (width 0.2) (layer "F.Cu") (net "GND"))
 (segment (start 113.45 46.23) (end 114.6017 46.23) (width 0.2) (layer "F.Cu") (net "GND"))
 (segment (start 141.1215 47.3817) (end 140.0017 48.5015) (width 0.2) (layer "F.Cu") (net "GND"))
 (segment (start 117.3783 48.77) (end 117.3783 48.482) (width 0.2) (layer "F.Cu") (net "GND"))
 (segment (start 155.4783 48.482) (end 154.6146 47.6183) (width 0.2) (layer "F.Cu") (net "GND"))
 (segment (start 149.01 46.23) (end 150.1617 46.23) (width 0.2) (layer "F.Cu") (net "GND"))
 (segment (start 149.01 46.23) (end 147.8583 46.23) (width 0.2) (layer "F.Cu") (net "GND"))
 (segment (start 118.53 48.77) (end 117.3783 48.77) (width 0.2) (layer "F.Cu") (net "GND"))
 (segment (start 125.6724 45.0508) (end 124.7617 45.9615) (width 0.2) (layer "F.Cu") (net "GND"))
 (segment (start 141.9146 47.3817) (end 141.1215 47.3817) (width 0.2) (layer "F.Cu") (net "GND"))
 (segment (start 140.0017 48.5015) (end 140.0017 48.77) (width 0.2) (layer "F.Cu") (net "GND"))
 (segment (start 123.61 46.23) (end 122.4583 46.23) (width 0.2) (layer "F.Cu") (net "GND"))
 (segment (start 120.8015 47.3817) (end 119.6817 48.5015) (width 0.2) (layer "F.Cu") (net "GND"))
 (segment (start 143.8917 53.2583) (end 144 53.15) (width 0.2) (layer "F.Cu") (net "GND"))
 (segment (start 132.3817 46.518) (end 133.2454 47.3817) (width 0.2) (layer "F.Cu") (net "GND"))
 (segment (start 143.93 46.23) (end 142.7783 46.23) (width 0.2) (layer "F.Cu") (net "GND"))
 (segment (start 132.3817 46.23) (end 132.3817 46.518) (width 0.2) (layer "F.Cu") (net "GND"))
 (segment (start 130.0783 46.23) (end 130.0783 45.9421) (width 0.2) (layer "F.Cu") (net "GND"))
 (via (at 143.8917 53.2583) (size 0.6) (drill 0.3) (layers "F.Cu" "B.Cu") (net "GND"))
 (segment (start 143.93 47.3817) (end 144.2179 47.3817) (width 0.2) (layer "B.Cu") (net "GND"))
 (segment (start 144.2179 47.3817) (end 145.1206 48.2844) (width 0.2) (layer "B.Cu") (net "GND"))
 (segment (start 145.1206 48.2844) (end 145.1206 52.0294) (width 0.2) (layer "B.Cu") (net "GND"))
 (segment (start 145.1206 52.0294) (end 143.8917 53.2583) (width 0.2) (layer "B.Cu") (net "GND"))
 (segment (start 143.93 46.23) (end 143.93 47.3817) (width 0.2) (layer "B.Cu") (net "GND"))
 (segment (start 138.65 56.5) (end 138.9559 56.5) (width 0.2) (layer "F.Cu") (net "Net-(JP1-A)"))
 (segment (start 138.9559 56.5) (end 140.1517 55.3042) (width 0.2) (layer "F.Cu") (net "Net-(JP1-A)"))
 (segment (start 140.1517 55.3042) (end 140.8558 55.3042) (width 0.2) (layer "F.Cu") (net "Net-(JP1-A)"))
 (segment (start 140.8558 55.3042) (end 141.525 54.635) (width 0.2) (layer "F.Cu") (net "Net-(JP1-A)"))
 (segment (start 110.91 46.23) (end 108.37 46.23) (width 0.2) (layer "F.Cu") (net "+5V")))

